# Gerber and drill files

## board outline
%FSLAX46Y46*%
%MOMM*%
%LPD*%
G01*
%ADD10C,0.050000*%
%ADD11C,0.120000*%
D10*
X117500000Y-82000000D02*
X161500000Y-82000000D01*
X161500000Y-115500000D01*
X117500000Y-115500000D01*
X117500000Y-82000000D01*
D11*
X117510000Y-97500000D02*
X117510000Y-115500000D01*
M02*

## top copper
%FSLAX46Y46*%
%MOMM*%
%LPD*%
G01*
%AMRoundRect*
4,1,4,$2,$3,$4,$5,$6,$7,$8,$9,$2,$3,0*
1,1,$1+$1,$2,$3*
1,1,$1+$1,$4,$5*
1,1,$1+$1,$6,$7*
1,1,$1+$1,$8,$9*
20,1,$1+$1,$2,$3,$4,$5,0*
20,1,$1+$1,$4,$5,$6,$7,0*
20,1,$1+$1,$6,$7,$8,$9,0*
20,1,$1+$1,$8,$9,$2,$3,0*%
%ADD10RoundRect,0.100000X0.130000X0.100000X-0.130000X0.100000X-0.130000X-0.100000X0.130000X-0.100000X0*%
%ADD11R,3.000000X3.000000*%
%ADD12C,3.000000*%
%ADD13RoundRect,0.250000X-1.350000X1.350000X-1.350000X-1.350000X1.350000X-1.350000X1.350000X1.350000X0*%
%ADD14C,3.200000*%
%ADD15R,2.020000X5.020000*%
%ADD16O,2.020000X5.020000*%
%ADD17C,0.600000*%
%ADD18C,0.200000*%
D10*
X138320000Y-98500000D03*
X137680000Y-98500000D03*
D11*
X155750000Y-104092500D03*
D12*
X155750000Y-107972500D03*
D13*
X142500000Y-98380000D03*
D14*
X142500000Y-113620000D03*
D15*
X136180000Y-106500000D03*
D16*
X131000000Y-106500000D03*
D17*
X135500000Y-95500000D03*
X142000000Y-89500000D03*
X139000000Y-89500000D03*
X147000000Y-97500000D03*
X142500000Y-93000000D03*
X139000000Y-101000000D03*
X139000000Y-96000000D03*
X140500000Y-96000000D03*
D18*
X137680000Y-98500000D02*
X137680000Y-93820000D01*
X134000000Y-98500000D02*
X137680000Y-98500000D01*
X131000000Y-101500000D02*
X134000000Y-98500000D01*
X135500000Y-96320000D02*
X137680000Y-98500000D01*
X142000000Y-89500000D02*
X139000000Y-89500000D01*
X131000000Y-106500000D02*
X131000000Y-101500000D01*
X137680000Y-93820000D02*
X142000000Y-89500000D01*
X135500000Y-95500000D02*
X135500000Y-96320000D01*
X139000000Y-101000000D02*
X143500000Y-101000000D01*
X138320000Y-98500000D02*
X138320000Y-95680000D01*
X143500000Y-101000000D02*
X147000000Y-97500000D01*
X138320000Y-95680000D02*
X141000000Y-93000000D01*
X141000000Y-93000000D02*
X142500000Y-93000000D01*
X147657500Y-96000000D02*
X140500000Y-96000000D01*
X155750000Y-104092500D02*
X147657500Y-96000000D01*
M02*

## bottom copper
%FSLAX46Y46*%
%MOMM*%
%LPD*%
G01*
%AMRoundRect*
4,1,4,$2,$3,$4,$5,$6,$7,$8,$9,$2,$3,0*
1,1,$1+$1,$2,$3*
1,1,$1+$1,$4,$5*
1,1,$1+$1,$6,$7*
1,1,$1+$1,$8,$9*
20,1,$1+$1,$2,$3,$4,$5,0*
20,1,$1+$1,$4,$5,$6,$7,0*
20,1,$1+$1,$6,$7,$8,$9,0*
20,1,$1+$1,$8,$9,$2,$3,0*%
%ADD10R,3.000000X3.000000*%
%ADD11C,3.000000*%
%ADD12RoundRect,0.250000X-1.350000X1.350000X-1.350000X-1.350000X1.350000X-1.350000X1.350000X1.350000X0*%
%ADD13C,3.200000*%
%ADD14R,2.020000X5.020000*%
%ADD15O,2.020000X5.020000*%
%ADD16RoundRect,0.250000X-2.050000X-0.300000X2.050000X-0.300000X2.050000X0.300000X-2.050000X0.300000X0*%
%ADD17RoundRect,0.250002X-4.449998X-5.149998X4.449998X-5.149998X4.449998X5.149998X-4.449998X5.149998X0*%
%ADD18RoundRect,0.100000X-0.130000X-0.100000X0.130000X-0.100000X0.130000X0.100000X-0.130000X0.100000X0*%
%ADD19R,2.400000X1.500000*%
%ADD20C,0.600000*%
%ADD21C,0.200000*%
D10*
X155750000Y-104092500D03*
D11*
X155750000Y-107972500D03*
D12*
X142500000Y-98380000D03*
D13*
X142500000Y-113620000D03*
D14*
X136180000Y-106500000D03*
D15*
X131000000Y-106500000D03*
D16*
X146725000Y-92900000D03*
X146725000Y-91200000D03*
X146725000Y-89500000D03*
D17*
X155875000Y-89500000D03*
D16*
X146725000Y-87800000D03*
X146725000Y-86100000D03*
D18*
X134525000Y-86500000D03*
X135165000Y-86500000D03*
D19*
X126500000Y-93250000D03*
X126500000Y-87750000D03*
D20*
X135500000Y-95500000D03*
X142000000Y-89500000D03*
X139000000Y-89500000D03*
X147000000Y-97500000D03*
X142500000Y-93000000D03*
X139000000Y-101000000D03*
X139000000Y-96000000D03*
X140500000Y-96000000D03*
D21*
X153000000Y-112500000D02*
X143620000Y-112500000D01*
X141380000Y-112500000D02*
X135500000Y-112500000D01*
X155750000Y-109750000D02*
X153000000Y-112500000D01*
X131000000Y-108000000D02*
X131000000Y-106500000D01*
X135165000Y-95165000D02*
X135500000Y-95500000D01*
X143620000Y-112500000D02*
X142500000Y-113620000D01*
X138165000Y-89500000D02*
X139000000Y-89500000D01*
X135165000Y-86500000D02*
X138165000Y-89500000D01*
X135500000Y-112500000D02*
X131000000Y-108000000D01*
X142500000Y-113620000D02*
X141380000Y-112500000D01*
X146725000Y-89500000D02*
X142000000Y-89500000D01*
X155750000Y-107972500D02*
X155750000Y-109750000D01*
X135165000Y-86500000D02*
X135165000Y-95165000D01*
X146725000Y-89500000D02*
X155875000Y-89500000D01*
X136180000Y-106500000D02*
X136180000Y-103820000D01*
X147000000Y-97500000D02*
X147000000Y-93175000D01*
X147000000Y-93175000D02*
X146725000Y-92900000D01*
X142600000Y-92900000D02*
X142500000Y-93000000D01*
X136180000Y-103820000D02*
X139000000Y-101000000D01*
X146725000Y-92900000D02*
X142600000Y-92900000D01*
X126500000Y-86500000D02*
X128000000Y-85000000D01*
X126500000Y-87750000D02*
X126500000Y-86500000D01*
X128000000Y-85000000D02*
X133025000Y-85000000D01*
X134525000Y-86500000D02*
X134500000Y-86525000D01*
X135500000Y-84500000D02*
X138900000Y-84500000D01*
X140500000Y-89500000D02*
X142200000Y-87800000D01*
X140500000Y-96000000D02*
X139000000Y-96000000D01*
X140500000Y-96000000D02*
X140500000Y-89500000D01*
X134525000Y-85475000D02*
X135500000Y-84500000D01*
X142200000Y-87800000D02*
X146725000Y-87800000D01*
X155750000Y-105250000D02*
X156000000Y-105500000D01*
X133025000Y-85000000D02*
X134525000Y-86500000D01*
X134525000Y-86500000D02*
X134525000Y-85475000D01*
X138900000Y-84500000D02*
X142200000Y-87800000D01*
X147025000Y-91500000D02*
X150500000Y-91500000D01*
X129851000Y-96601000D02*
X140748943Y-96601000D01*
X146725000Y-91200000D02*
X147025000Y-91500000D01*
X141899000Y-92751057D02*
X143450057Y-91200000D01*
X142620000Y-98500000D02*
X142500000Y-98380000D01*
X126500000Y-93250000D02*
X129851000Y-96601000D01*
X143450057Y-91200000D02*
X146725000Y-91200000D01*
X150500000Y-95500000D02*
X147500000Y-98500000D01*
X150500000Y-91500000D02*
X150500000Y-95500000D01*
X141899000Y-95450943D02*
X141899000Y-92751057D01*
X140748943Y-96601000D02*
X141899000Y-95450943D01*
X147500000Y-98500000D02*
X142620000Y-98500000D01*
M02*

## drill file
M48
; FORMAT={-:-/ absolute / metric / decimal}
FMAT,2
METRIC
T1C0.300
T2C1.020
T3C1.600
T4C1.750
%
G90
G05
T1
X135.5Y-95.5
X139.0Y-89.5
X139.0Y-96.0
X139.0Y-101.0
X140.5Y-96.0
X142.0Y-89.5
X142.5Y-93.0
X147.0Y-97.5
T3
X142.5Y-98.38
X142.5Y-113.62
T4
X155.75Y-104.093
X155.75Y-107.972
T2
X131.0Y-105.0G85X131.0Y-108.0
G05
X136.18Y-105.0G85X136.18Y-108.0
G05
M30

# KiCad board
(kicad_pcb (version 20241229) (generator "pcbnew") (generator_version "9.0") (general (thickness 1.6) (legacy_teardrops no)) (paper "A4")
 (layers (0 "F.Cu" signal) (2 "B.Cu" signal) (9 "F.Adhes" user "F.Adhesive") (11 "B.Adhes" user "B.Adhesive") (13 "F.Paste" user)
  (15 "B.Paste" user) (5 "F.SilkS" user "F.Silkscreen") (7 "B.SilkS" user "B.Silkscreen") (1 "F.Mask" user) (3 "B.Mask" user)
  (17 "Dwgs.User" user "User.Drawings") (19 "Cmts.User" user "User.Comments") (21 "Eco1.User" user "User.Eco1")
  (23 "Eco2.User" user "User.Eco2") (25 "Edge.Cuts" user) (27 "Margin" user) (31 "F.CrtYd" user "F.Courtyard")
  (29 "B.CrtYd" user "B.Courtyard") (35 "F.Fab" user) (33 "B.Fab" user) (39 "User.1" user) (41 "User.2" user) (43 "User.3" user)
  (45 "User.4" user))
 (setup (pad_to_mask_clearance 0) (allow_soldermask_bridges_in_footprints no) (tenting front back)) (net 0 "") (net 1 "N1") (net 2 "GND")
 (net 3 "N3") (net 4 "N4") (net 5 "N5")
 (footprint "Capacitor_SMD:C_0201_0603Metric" (layer "F.Cu") (at 138 98.5 180)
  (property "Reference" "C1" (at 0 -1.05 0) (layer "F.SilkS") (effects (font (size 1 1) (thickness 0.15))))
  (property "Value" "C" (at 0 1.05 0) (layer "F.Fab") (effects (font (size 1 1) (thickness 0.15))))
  (pad "" smd roundrect (at -0.345 0 180) (size 0.318 0.36) (layers "F.Paste") (roundrect_rratio 0.25))
  (pad "" smd roundrect (at 0.345 0 180) (size 0.318 0.36) (layers "F.Paste") (roundrect_rratio 0.25))
  (pad "1" smd roundrect (at -0.32 0 180) (size 0.46 0.4) (layers "F.Cu" "F.Mask") (roundrect_rratio 0.25) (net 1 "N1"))
  (pad "2" smd roundrect (at 0.32 0 180) (size 0.46 0.4) (layers "F.Cu" "F.Mask") (roundrect_rratio 0.25) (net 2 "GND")))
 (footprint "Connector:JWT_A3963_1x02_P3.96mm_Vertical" (layer "F.Cu") (at 155.75 104.0925 -90)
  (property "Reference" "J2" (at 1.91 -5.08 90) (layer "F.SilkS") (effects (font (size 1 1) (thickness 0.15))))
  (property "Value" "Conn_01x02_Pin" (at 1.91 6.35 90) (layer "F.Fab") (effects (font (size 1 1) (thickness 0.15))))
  (pad "1" thru_hole rect (at 0 0 270) (size 3 3) (drill 1.75) (layers "*.Cu" "*.Mask") (remove_unused_layers no) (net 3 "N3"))
  (pad "2" thru_hole circle (at 3.88 0 270) (size 3 3) (drill 1.75) (layers "*.Cu" "*.Mask") (remove_unused_layers no) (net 2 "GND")))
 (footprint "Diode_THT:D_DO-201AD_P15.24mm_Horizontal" (layer "F.Cu") (at 142.5 98.38 -90)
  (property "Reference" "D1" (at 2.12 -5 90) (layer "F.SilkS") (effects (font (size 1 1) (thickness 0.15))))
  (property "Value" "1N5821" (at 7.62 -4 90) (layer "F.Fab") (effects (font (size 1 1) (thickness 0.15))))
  (pad "1" thru_hole roundrect (at 0 0 270) (size 3.2 3.2) (drill 1.6) (layers "*.Cu" "*.Mask") (remove_unused_layers no)
   (roundrect_rratio 0.078125) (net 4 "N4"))
  (pad "2" thru_hole circle (at 15.24 0 270) (size 3.2 3.2) (drill 1.6) (layers "*.Cu" "*.Mask") (remove_unused_layers no) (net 2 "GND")))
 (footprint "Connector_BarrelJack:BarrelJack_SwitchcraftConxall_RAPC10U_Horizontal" (layer "F.Cu") (at 136.18 106.5)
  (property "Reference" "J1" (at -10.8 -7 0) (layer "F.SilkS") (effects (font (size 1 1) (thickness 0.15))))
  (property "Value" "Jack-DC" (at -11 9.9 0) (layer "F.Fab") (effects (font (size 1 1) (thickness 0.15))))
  (fp_line (start -18.67 -9) (end -18.67 9) (stroke (width 0.12) (type solid)) (layer "Edge.Cuts"))
  (pad "1" thru_hole rect (at 0 0) (size 2.02 5.02) (drill oval 1.02 4.02) (layers "*.Cu" "*.Mask") (remove_unused_layers no) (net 1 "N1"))
  (pad "2" thru_hole oval (at -5.18 0) (size 2.02 5.02) (drill oval 1.02 4.02) (layers "*.Cu" "*.Mask") (remove_unused_layers no)
   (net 2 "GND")))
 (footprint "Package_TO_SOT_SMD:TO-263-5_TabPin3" (layer "B.Cu") (at 154.375 89.5)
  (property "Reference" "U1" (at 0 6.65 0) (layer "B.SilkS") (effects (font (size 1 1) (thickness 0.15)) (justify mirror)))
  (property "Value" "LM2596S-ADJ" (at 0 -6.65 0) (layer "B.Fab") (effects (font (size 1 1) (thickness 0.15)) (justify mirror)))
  (pad "" smd roundrect (at -0.925 -2.775) (size 4.55 5.25) (layers "B.Paste") (roundrect_rratio 0.054945))
  (pad "" smd roundrect (at -0.925 2.775) (size 4.55 5.25) (layers "B.Paste") (roundrect_rratio 0.054945))
  (pad "" smd roundrect (at 3.925 -2.775) (size 4.55 5.25) (layers "B.Paste") (roundrect_rratio 0.054945))
  (pad "" smd roundrect (at 3.925 2.775) (size 4.55 5.25) (layers "B.Paste") (roundrect_rratio 0.054945))
  (pad "1" smd roundrect (at -7.65 3.4) (size 4.6 1.1) (layers "B.Cu" "B.Mask" "B.Paste") (roundrect_rratio 0.227273) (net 1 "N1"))
  (pad "2" smd roundrect (at -7.65 1.7) (size 4.6 1.1) (layers "B.Cu" "B.Mask" "B.Paste") (roundrect_rratio 0.227273) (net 4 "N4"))
  (pad "3" smd roundrect (at -7.65 0) (size 4.6 1.1) (layers "B.Cu" "B.Mask" "B.Paste") (roundrect_rratio 0.227273) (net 2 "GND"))
  (pad "3" smd roundrect (at 1.5 0) (size 9.4 10.8) (layers "B.Cu" "B.Mask") (roundrect_rratio 0.026596) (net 2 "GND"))
  (pad "4" smd roundrect (at -7.65 -1.7) (size 4.6 1.1) (layers "B.Cu" "B.Mask" "B.Paste") (roundrect_rratio 0.227273) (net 3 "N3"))
  (pad "5" smd roundrect (at -7.65 -3.4) (size 4.6 1.1) (layers "B.Cu" "B.Mask" "B.Paste") (roundrect_rratio 0.227273) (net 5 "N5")))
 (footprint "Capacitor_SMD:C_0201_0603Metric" (layer "B.Cu") (at 134.845 86.5)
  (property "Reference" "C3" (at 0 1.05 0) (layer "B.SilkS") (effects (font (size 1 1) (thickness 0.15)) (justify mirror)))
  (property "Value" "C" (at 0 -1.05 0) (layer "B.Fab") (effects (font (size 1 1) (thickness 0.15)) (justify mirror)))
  (pad "" smd roundrect (at -0.345 0) (size 0.318 0.36) (layers "B.Paste") (roundrect_rratio 0.25))
  (pad "" smd roundrect (at 0.345 0) (size 0.318 0.36) (layers "B.Paste") (roundrect_rratio 0.25))
  (pad "1" smd roundrect (at -0.32 0) (size 0.46 0.4) (layers "B.Cu" "B.Mask") (roundrect_rratio 0.25) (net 3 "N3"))
  (pad "2" smd roundrect (at 0.32 0) (size 0.46 0.4) (layers "B.Cu" "B.Mask") (roundrect_rratio 0.25) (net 2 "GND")))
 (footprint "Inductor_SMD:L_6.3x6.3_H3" (layer "B.Cu") (at 126.5 90.5 90)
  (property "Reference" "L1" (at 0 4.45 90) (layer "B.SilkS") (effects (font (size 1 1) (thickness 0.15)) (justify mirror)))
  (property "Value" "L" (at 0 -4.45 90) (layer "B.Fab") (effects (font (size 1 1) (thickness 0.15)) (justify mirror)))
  (pad "1" smd rect (at -2.75 0 90) (size 1.5 2.4) (layers "B.Cu" "B.Mask" "B.Paste") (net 4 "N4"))
  (pad "2" smd rect (at 2.75 0 90) (size 1.5 2.4) (layers "B.Cu" "B.Mask" "B.Paste") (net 3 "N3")))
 (gr_rect (start 117.5 82) (end 161.5 115.5) (stroke (width 0.05) (type default)) (fill no) (layer "Edge.Cuts"))
 (segment (start 137.68 98.5) (end 137.68 93.82) (width 0.2) (layer "F.Cu") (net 2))
 (segment (start 134 98.5) (end 137.68 98.5) (width 0.2) (layer "F.Cu") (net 2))
 (segment (start 131 101.5) (end 134 98.5) (width 0.2) (layer "F.Cu") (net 2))
 (segment (start 135.5 96.32) (end 137.68 98.5) (width 0.2) (layer "F.Cu") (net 2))
 (segment (start 142 89.5) (end 139 89.5) (width 0.2) (layer "F.Cu") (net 2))
 (segment (start 131 106.5) (end 131 101.5) (width 0.2) (layer "F.Cu") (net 2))
 (segment (start 137.68 93.82) (end 142 89.5) (width 0.2) (layer "F.Cu") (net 2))
 (segment (start 135.5 95.5) (end 135.5 96.32) (width 0.2) (layer "F.Cu") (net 2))
 (via (at 135.5 95.5) (size 0.6) (drill 0.3) (layers "F.Cu" "B.Cu") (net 2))
 (via (at 142 89.5) (size 0.6) (drill 0.3) (layers "F.Cu" "B.Cu") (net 2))
 (via (at 139 89.5) (size 0.6) (drill 0.3) (layers "F.Cu" "B.Cu") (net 2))
 (segment (start 153 112.5) (end 143.62 112.5) (width 0.2) (layer "B.Cu") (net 2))
 (segment (start 141.38 112.5) (end 135.5 112.5) (width 0.2) (layer "B.Cu") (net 2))
 (segment (start 155.75 109.75) (end 153 112.5) (width 0.2) (layer "B.Cu") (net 2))
 (segment (start 131 108) (end 131 106.5) (width 0.2) (layer "B.Cu") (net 2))
 (segment (start 135.165 95.165) (end 135.5 95.5) (width 0.2) (layer "B.Cu") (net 2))
 (segment (start 143.62 112.5) (end 142.5 113.62) (width 0.2) (layer "B.Cu") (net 2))
 (segment (start 138.165 89.5) (end 139 89.5) (width 0.2) (layer "B.Cu") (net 2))
 (segment (start 135.165 86.5) (end 138.165 89.5) (width 0.2) (layer "B.Cu") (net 2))
 (segment (start 135.5 112.5) (end 131 108) (width 0.2) (layer "B.Cu") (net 2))
 (segment (start 142.5 113.62) (end 141.38 112.5) (width 0.2) (layer "B.Cu") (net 2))
 (segment (start 146.725 89.5) (end 142 89.5) (width 0.2) (layer "B.Cu") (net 2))
 (segment (start 155.75 107.9725) (end 155.75 109.75) (width 0.2) (layer "B.Cu") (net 2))
 (segment (start 135.165 86.5) (end 135.165 95.165) (width 0.2) (layer "B.Cu") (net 2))
 (segment (start 146.725 89.5) (end 155.875 89.5) (width 0.2) (layer "B.Cu") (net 2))
 (segment (start 139 101) (end 143.5 101) (width 0.2) (layer "F.Cu") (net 1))
 (segment (start 138.32 98.5) (end 138.32 95.68) (width 0.2) (layer "F.Cu") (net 1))
 (segment (start 143.5 101) (end 147 97.5) (width 0.2) (layer "F.Cu") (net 1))
 (segment (start 138.32 95.68) (end 141 93) (width 0.2) (layer "F.Cu") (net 1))
 (segment (start 141 93) (end 142.5 93) (width 0.2) (layer "F.Cu") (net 1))
 (via (at 147 97.5) (size 0.6) (drill 0.3) (layers "F.Cu" "B.Cu") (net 1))
 (via (at 142.5 93) (size 0.6) (drill 0.3) (layers "F.Cu" "B.Cu") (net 1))
 (via (at 139 101) (size 0.6) (drill 0.3) (layers "F.Cu" "B.Cu") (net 1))
 (segment (start 136.18 106.5) (end 136.18 103.82) (width 0.2) (layer "B.Cu") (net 1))
 (segment (start 147 97.5) (end 147 93.175) (width 0.2) (layer "B.Cu") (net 1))
 (segment (start 147 93.175) (end 146.725 92.9) (width 0.2) (layer "B.Cu") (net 1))
 (segment (start 142.6 92.9) (end 142.5 93) (width 0.2) (layer "B.Cu") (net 1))
 (segment (start 136.18 103.82) (end 139 101) (width 0.2) (layer "B.Cu") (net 1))
 (segment (start 146.725 92.9) (end 142.6 92.9) (width 0.2) (layer "B.Cu") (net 1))
 (segment (start 147.6575 96) (end 140.5 96) (width 0.2) (layer "F.Cu") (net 3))
 (segment (start 155.75 104.0925) (end 147.6575 96) (width 0.2) (layer "F.Cu") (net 3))
 (via (at 139 96) (size 0.6) (drill 0.3) (layers "F.Cu" "B.Cu") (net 3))
 (via (at 140.5 96) (size 0.6) (drill 0.3) (layers "F.Cu" "B.Cu") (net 3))
 (segment (start 126.5 86.5) (end 128 85) (width 0.2) (layer "B.Cu") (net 3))
 (segment (start 126.5 87.75) (end 126.5 86.5) (width 0.2) (layer "B.Cu") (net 3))
 (segment (start 128 85) (end 133.025 85) (width 0.2) (layer "B.Cu") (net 3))
 (segment (start 134.525 86.5) (end 134.5 86.525) (width 0.2) (layer "B.Cu") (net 3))
 (segment (start 135.5 84.5) (end 138.9 84.5) (width 0.2) (layer "B.Cu") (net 3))
 (segment (start 140.5 89.5) (end 142.2 87.8) (width 0.2) (layer "B.Cu") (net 3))
 (segment (start 140.5 96) (end 139 96) (width 0.2) (layer "B.Cu") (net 3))
 (segment (start 140.5 96) (end 140.5 89.5) (width 0.2) (layer "B.Cu") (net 3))
 (segment (start 134.525 85.475) (end 135.5 84.5) (width 0.2) (layer "B.Cu") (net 3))
 (segment (start 142.2 87.8) (end 146.725 87.8) (width 0.2) (layer "B.Cu") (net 3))
 (segment (start 155.75 105.25) (end 156 105.5) (width 0.2) (layer "B.Cu") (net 3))
 (segment (start 133.025 85) (end 134.525 86.5) (width 0.2) (layer "B.Cu") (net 3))
 (segment (start 134.525 86.5) (end 134.525 85.475) (width 0.2) (layer "B.Cu") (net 3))
 (segment (start 138.9 84.5) (end 142.2 87.8) (width 0.2) (layer "B.Cu") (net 3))
 (segment (start 147.025 91.5) (end 150.5 91.5) (width 0.2) (layer "B.Cu") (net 4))
 (segment (start 129.851 96.601) (end 140.748943 96.601) (width 0.2) (layer "B.Cu") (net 4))
 (segment (start 146.725 91.2) (end 147.025 91.5) (width 0.2) (layer "B.Cu") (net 4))
 (segment (start 141.899 92.751057) (end 143.450057 91.2) (width 0.2) (layer "B.Cu") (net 4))
 (segment (start 142.62 98.5) (end 142.5 98.38) (width 0.2) (layer "B.Cu") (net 4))
 (segment (start 126.5 93.25) (end 129.851 96.601) (width 0.2) (layer "B.Cu") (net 4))
 (segment (start 143.450057 91.2) (end 146.725 91.2) (width 0.2) (layer "B.Cu") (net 4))
 (segment (start 150.5 95.5) (end 147.5 98.5) (width 0.2) (layer "B.Cu") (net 4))
 (segment (start 150.5 91.5) (end 150.5 95.5) (width 0.2) (layer "B.Cu") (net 4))
 (segment (start 141.899 95.450943) (end 141.899 92.751057) (width 0.2) (layer "B.Cu") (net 4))
 (segment (start 140.748943 96.601) (end 141.899 95.450943) (width 0.2) (layer "B.Cu") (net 4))
 (segment (start 147.5 98.5) (end 142.62 98.5) (width 0.2) (layer "B.Cu") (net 4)))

